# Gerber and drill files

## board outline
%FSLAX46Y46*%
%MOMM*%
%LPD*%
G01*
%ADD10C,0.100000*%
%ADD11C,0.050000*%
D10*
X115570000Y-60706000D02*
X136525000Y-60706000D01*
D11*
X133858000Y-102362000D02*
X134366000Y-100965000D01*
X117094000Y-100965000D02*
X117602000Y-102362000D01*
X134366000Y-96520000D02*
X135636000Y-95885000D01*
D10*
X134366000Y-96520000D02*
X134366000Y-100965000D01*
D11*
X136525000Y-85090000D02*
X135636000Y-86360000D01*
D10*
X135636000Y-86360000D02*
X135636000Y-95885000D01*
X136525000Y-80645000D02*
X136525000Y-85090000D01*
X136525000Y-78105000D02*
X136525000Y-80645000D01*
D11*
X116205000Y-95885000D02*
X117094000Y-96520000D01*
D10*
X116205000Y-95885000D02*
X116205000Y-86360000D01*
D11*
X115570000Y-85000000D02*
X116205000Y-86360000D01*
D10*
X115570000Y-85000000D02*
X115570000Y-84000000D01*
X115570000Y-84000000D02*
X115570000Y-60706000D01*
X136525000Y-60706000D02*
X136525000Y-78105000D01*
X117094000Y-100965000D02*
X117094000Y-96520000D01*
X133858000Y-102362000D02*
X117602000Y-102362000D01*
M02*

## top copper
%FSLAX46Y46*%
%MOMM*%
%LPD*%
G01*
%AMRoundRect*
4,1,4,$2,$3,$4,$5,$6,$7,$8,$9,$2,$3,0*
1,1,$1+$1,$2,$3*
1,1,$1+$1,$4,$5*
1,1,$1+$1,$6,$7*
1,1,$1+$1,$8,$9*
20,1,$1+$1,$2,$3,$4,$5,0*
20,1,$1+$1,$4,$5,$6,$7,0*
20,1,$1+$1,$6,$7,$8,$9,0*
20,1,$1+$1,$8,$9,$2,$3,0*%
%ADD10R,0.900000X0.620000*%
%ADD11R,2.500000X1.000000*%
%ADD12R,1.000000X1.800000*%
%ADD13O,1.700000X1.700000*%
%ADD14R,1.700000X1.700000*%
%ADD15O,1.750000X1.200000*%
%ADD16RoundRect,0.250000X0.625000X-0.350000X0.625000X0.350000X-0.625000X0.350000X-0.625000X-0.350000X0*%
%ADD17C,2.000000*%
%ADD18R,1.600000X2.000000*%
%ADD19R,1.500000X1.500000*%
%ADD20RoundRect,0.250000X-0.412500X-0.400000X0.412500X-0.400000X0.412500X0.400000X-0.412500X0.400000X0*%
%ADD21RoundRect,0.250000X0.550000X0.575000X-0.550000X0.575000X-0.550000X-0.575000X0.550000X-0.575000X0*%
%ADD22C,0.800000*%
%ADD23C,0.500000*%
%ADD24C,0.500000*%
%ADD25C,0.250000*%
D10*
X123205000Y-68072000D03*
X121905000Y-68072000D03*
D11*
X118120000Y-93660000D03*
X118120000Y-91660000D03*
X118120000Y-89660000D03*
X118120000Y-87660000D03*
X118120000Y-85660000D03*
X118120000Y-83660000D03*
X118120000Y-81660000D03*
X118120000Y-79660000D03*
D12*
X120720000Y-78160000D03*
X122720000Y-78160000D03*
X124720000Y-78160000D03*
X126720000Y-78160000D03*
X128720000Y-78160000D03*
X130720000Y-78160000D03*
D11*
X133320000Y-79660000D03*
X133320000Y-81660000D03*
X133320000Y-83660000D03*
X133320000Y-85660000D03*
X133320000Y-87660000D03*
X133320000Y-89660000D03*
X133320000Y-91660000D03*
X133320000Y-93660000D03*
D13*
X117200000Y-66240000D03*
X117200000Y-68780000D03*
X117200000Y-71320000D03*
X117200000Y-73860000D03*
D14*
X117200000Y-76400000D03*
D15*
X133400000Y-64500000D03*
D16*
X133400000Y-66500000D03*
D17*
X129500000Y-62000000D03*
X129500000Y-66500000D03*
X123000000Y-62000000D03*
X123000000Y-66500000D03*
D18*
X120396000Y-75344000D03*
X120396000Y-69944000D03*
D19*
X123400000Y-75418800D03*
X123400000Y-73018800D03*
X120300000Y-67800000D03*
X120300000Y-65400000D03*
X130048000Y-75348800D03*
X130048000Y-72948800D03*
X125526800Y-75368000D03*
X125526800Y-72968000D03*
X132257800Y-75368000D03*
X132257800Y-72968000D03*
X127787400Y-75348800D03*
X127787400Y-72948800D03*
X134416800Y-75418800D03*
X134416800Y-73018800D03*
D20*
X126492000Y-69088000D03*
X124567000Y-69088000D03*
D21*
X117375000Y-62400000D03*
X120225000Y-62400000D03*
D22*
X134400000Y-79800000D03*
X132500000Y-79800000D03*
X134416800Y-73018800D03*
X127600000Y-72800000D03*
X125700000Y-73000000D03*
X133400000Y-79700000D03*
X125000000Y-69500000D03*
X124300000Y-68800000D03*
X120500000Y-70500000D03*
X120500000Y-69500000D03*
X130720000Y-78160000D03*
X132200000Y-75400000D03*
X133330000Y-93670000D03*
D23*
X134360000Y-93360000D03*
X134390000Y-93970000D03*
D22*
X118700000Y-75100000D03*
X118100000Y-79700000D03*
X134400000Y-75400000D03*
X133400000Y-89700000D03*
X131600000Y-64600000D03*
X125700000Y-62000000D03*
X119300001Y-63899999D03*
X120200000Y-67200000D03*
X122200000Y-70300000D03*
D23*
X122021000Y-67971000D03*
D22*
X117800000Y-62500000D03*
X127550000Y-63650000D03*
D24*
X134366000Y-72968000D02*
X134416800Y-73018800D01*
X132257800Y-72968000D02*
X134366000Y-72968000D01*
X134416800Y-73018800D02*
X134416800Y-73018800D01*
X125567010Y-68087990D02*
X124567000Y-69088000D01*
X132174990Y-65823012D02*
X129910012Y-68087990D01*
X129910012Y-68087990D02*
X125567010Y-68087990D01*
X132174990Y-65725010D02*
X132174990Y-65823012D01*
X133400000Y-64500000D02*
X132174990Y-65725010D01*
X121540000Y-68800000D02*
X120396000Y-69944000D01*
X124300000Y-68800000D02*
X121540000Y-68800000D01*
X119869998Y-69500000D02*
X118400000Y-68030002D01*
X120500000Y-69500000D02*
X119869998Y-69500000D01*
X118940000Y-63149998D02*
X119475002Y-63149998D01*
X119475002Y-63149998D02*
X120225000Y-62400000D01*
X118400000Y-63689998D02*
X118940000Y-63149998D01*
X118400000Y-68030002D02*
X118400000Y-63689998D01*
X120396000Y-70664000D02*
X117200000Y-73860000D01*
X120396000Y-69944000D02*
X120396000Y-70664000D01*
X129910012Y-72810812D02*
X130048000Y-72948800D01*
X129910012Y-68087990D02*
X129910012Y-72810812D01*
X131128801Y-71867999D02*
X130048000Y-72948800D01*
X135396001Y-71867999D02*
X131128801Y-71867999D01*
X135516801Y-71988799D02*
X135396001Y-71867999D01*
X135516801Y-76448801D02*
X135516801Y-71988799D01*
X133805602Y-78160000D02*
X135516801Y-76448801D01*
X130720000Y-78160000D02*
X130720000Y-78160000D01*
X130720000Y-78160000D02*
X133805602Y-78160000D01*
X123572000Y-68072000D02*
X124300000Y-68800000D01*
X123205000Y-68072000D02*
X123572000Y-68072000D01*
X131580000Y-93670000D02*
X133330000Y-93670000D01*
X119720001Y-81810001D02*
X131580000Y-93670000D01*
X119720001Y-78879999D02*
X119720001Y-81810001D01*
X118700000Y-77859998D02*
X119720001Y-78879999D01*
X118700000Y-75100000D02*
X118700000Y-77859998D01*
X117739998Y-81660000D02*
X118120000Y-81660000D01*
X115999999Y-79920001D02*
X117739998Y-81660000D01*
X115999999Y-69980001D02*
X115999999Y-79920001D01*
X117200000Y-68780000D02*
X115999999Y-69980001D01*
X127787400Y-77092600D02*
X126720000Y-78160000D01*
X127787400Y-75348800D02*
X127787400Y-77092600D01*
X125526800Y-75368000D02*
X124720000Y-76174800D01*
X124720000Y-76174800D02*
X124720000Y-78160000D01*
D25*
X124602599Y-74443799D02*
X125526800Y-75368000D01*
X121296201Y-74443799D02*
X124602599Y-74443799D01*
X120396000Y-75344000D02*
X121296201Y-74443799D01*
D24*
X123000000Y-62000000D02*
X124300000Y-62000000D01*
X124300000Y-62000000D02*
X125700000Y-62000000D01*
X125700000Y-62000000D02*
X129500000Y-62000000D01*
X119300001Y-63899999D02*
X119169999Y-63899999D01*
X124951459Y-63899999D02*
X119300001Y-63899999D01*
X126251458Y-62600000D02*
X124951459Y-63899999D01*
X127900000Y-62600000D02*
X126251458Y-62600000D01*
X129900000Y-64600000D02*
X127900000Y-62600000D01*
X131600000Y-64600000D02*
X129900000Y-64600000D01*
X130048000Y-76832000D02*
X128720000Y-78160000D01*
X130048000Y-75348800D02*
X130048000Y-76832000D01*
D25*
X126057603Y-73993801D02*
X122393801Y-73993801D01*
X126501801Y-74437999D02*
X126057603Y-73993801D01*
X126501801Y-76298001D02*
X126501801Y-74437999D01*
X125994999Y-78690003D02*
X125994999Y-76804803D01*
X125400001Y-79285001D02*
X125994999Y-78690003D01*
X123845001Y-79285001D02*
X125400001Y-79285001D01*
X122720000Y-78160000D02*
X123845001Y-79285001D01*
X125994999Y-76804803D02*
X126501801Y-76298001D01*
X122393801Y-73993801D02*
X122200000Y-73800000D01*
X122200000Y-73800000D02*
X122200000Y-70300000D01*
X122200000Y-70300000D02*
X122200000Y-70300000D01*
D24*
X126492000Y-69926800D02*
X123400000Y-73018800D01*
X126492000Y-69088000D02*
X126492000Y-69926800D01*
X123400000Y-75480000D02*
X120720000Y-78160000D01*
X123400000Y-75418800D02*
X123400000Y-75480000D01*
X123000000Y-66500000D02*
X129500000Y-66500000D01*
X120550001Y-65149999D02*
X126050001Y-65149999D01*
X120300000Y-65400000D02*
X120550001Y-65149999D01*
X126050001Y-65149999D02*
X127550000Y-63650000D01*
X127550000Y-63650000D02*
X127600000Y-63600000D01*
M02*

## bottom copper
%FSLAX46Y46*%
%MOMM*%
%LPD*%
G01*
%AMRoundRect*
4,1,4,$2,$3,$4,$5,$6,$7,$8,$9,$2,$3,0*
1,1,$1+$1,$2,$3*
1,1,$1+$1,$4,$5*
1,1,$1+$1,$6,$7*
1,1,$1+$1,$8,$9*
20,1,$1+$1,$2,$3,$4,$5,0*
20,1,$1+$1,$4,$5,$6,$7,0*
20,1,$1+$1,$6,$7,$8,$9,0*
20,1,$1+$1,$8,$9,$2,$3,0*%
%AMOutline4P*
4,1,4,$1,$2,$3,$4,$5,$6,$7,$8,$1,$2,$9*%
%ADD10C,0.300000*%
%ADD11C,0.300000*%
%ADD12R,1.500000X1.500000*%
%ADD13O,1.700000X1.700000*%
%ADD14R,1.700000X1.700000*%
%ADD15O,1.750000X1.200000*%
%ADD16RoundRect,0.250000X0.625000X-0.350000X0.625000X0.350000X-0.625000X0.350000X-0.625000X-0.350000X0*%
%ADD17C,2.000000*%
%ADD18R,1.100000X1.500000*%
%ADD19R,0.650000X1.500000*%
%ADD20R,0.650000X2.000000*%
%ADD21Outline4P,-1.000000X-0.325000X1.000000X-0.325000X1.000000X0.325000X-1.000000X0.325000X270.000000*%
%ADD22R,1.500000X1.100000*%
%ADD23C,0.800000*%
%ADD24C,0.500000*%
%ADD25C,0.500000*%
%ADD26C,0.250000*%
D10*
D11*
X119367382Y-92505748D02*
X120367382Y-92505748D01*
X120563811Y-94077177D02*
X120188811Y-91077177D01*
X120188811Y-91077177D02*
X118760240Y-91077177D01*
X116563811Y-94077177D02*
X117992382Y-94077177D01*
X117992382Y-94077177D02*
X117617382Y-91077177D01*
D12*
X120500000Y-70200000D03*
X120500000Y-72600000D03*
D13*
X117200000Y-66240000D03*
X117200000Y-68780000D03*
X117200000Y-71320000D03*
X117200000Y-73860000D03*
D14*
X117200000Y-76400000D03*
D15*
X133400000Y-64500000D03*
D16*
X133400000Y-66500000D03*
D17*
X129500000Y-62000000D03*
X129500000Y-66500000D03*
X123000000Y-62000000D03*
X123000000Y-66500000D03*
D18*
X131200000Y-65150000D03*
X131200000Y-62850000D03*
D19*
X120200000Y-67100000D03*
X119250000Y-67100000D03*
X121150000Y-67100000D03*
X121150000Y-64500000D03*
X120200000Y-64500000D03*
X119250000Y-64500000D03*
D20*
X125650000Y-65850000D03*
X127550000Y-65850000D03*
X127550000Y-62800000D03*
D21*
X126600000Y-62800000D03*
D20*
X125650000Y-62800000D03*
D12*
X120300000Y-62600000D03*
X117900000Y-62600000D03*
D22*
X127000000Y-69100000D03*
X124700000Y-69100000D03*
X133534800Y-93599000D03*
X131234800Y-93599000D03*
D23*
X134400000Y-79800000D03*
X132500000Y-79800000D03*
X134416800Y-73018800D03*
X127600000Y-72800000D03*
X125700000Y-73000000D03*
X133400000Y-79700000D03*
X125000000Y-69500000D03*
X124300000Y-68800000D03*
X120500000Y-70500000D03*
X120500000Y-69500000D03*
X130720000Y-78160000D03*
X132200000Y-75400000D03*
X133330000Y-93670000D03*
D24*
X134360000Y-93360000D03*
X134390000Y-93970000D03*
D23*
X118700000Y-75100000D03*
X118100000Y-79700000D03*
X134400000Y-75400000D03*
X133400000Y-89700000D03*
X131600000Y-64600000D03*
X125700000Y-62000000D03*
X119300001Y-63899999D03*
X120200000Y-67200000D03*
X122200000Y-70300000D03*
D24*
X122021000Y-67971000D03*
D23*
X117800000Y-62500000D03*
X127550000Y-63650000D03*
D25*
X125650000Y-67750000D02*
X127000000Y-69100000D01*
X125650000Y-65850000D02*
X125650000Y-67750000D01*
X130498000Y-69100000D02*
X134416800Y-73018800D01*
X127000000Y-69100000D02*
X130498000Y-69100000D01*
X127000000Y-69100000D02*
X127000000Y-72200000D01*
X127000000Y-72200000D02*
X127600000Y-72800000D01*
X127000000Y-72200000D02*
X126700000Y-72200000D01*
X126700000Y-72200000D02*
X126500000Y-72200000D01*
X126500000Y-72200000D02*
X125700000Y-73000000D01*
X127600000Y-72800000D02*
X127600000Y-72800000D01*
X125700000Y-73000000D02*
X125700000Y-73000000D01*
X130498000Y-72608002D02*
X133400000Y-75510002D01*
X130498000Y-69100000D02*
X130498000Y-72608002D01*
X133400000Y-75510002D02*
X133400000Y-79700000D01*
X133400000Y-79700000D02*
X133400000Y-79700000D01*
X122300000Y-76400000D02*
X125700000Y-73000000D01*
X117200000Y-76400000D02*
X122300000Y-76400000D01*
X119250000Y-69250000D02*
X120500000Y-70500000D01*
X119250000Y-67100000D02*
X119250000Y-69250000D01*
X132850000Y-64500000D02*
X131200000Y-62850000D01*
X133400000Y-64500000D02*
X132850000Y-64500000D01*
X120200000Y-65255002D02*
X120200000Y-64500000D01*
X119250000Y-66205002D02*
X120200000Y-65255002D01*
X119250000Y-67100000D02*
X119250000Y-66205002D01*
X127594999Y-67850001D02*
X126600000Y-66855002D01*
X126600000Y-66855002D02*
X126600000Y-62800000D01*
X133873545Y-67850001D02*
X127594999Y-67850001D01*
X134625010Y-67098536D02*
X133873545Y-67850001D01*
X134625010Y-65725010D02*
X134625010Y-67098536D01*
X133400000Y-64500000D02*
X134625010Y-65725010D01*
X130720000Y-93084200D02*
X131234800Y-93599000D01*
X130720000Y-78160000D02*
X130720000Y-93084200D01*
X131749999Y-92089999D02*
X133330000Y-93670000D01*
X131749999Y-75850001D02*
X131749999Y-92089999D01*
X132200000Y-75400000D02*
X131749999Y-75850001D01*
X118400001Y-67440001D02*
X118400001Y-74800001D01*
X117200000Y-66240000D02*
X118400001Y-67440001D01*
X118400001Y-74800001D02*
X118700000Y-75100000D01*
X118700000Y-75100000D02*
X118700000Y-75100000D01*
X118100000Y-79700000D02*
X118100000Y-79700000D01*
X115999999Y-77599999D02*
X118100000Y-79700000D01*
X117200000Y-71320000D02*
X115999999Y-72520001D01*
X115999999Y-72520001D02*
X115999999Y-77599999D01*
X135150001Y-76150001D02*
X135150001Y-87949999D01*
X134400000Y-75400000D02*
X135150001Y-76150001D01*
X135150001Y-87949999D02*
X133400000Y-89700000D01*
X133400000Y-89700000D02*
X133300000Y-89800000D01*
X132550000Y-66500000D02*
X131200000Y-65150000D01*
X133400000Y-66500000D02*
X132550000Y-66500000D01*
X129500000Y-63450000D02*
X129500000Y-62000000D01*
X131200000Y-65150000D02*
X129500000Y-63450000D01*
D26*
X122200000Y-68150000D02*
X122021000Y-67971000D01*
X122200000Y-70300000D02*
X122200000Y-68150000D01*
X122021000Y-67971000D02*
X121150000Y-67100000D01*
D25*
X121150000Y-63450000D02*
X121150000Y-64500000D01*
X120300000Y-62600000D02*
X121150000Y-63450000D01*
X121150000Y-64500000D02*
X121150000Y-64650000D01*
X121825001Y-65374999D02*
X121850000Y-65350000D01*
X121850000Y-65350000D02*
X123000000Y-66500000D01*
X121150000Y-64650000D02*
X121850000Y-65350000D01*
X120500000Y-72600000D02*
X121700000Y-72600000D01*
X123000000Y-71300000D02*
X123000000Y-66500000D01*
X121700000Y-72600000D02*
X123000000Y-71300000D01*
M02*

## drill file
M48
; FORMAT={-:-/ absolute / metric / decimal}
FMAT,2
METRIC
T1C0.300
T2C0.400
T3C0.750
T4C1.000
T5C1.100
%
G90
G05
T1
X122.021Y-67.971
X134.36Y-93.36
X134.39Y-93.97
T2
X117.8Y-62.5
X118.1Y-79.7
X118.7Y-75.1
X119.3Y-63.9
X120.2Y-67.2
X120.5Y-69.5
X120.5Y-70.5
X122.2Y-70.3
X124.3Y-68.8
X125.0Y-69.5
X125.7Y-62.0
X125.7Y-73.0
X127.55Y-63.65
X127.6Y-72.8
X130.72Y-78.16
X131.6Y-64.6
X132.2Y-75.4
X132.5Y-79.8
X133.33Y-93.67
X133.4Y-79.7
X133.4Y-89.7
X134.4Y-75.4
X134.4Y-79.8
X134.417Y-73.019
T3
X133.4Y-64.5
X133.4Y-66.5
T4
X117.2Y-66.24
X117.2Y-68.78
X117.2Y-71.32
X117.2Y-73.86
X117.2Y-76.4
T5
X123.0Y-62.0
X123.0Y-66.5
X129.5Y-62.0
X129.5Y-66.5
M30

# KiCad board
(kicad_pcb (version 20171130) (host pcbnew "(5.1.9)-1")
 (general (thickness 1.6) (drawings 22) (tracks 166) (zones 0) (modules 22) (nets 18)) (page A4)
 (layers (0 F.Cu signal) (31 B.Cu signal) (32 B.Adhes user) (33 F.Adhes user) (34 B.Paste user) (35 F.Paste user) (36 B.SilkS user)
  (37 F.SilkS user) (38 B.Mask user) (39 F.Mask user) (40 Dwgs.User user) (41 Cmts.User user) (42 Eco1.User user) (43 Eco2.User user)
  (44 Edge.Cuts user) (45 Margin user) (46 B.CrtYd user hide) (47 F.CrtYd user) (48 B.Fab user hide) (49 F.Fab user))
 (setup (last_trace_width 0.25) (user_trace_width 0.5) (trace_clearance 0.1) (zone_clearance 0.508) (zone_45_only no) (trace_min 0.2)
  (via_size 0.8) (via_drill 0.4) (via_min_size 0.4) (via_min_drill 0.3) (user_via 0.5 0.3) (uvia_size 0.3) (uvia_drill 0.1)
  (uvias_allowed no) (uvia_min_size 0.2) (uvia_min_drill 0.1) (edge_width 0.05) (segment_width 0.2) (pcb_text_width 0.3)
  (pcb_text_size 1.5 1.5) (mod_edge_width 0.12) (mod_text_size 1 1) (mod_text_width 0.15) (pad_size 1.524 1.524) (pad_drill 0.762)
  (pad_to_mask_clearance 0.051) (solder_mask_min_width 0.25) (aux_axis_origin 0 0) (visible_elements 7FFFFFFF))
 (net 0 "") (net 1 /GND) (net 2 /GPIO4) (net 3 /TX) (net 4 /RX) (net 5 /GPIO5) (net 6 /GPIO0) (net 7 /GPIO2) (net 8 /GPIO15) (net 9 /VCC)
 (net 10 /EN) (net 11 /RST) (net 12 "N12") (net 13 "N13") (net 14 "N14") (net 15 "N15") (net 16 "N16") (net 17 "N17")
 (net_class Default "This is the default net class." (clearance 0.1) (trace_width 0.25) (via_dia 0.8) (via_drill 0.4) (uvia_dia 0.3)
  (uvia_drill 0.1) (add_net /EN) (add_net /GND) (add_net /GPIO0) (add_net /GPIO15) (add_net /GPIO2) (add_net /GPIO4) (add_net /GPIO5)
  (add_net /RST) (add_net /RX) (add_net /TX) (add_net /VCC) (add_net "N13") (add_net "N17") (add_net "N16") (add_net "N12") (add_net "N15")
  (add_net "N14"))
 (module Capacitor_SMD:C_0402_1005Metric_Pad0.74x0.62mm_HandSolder (layer F.Cu) (at 122.555 68.072)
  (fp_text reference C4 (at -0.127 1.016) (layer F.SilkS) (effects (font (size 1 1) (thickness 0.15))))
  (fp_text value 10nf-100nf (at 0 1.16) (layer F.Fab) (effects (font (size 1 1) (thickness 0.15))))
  (pad 2 smd rect (at 0.65 0) (size 0.9 0.62) (layers F.Cu F.Paste F.Mask) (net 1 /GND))
  (pad 1 smd rect (at -0.65 0) (size 0.9 0.62) (layers F.Cu F.Paste F.Mask) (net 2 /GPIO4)))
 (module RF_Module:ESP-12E (layer F.Cu) (at 125.72 90.16 180)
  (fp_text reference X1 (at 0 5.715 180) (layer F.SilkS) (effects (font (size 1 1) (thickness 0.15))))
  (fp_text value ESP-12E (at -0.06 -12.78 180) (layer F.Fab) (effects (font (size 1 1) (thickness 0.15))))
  (pad 22 smd rect (at 7.6 -3.5 180) (size 2.5 1) (layers F.Cu F.Paste F.Mask))
  (pad 21 smd rect (at 7.6 -1.5 180) (size 2.5 1) (layers F.Cu F.Paste F.Mask))
  (pad 20 smd rect (at 7.6 0.5 180) (size 2.5 1) (layers F.Cu F.Paste F.Mask))
  (pad 19 smd rect (at 7.6 2.5 180) (size 2.5 1) (layers F.Cu F.Paste F.Mask))
  (pad 18 smd rect (at 7.6 4.5 180) (size 2.5 1) (layers F.Cu F.Paste F.Mask))
  (pad 17 smd rect (at 7.6 6.5 180) (size 2.5 1) (layers F.Cu F.Paste F.Mask))
  (pad 16 smd rect (at 7.6 8.5 180) (size 2.5 1) (layers F.Cu F.Paste F.Mask) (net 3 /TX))
  (pad 15 smd rect (at 7.6 10.5 180) (size 2.5 1) (layers F.Cu F.Paste F.Mask) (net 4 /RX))
  (pad 14 smd rect (at 5 12 180) (size 1 1.8) (layers F.Cu F.Paste F.Mask) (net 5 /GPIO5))
  (pad 13 smd rect (at 3 12 180) (size 1 1.8) (layers F.Cu F.Paste F.Mask) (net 2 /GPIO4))
  (pad 12 smd rect (at 1 12 180) (size 1 1.8) (layers F.Cu F.Paste F.Mask) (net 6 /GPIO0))
  (pad 11 smd rect (at -1 12 180) (size 1 1.8) (layers F.Cu F.Paste F.Mask) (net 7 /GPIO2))
  (pad 10 smd rect (at -3 12 180) (size 1 1.8) (layers F.Cu F.Paste F.Mask) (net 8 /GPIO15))
  (pad 9 smd rect (at -5 12 180) (size 1 1.8) (layers F.Cu F.Paste F.Mask) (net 1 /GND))
  (pad 8 smd rect (at -7.6 10.5 180) (size 2.5 1) (layers F.Cu F.Paste F.Mask) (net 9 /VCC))
  (pad 7 smd rect (at -7.6 8.5 180) (size 2.5 1) (layers F.Cu F.Paste F.Mask))
  (pad 6 smd rect (at -7.6 6.5 180) (size 2.5 1) (layers F.Cu F.Paste F.Mask))
  (pad 5 smd rect (at -7.6 4.5 180) (size 2.5 1) (layers F.Cu F.Paste F.Mask))
  (pad 4 smd rect (at -7.6 2.5 180) (size 2.5 1) (layers F.Cu F.Paste F.Mask))
  (pad 3 smd rect (at -7.6 0.5 180) (size 2.5 1) (layers F.Cu F.Paste F.Mask) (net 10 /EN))
  (pad 2 smd rect (at -7.6 -1.5 180) (size 2.5 1) (layers F.Cu F.Paste F.Mask))
  (pad 1 smd rect (at -7.6 -3.5 180) (size 2.5 1) (layers F.Cu F.Paste F.Mask) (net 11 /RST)))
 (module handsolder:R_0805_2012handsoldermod (layer B.Cu) (at 120.5 71.4 90)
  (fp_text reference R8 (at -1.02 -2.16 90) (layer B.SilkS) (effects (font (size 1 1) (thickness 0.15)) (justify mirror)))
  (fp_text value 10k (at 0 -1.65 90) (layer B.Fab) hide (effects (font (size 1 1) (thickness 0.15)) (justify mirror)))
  (pad 2 smd rect (at 1.2 0 90) (size 1.5 1.5) (layers B.Cu B.Paste B.Mask) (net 1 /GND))
  (pad 1 smd rect (at -1.2 0 90) (size 1.5 1.5) (layers B.Cu B.Paste B.Mask) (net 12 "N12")))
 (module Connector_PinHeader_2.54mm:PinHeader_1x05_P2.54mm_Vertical (layer F.Cu) (at 117.2 76.4 180)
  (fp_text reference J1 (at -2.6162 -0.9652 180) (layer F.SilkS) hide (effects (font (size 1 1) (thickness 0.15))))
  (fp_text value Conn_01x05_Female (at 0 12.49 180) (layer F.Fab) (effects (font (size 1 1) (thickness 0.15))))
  (pad 5 thru_hole oval (at 0 10.16 180) (size 1.7 1.7) (drill 1) (layers *.Cu *.Mask) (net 11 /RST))
  (pad 4 thru_hole oval (at 0 7.62 180) (size 1.7 1.7) (drill 1) (layers *.Cu *.Mask) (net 3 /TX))
  (pad 3 thru_hole oval (at 0 5.08 180) (size 1.7 1.7) (drill 1) (layers *.Cu *.Mask) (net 4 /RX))
  (pad 2 thru_hole oval (at 0 2.54 180) (size 1.7 1.7) (drill 1) (layers *.Cu *.Mask) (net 1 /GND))
  (pad 1 thru_hole rect (at 0 0 180) (size 1.7 1.7) (drill 1) (layers *.Cu *.Mask) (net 9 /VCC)))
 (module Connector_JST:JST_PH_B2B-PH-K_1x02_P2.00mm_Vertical (layer F.Cu) (at 133.4 66.5 90)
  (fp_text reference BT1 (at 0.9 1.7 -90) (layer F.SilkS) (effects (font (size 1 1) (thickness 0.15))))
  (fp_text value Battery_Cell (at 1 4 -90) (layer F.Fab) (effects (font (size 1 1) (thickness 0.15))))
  (pad 2 thru_hole oval (at 2 0 90) (size 1.2 1.75) (drill 0.75) (layers *.Cu *.Mask) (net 1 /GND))
  (pad 1 thru_hole roundrect (at 0 0 90) (size 1.2 1.75) (drill 0.75) (layers *.Cu *.Mask) (roundrect_rratio 0.208333) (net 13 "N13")))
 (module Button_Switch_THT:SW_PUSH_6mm (layer F.Cu) (at 123 62)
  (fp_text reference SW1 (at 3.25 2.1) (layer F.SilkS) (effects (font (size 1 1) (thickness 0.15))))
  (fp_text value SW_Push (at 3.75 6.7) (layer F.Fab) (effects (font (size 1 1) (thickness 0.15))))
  (pad 1 thru_hole circle (at 6.5 0 90) (size 2 2) (drill 1.1) (layers *.Cu *.Mask) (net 13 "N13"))
  (pad 2 thru_hole circle (at 6.5 4.5 90) (size 2 2) (drill 1.1) (layers *.Cu *.Mask) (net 12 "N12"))
  (pad 1 thru_hole circle (at 0 0 90) (size 2 2) (drill 1.1) (layers *.Cu *.Mask) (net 13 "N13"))
  (pad 2 thru_hole circle (at 0 4.5 90) (size 2 2) (drill 1.1) (layers *.Cu *.Mask) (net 12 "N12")))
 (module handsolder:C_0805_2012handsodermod (layer B.Cu) (at 131.2 64 270)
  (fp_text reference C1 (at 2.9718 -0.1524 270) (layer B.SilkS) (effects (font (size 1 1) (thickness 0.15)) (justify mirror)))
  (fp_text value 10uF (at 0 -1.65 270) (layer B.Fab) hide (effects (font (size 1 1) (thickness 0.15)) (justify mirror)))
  (pad 2 smd rect (at 1.15 0 270) (size 1.5 1.1) (layers B.Cu B.Paste B.Mask) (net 13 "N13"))
  (pad 1 smd rect (at -1.15 0 270) (size 1.5 1.1) (layers B.Cu B.Paste B.Mask) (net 1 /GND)))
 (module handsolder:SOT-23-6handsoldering (layer B.Cu) (at 120.2 65.8 270)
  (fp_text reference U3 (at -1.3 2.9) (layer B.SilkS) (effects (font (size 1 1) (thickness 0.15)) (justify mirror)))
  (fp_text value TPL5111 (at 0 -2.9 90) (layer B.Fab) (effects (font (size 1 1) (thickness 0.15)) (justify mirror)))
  (pad 5 smd rect (at 1.3 0 270) (size 1.5 0.65) (layers B.Cu B.Paste B.Mask) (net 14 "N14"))
  (pad 6 smd rect (at 1.3 0.95 270) (size 1.5 0.65) (layers B.Cu B.Paste B.Mask) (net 1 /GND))
  (pad 4 smd rect (at 1.3 -0.95 270) (size 1.5 0.65) (layers B.Cu B.Paste B.Mask) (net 2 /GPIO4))
  (pad 3 smd rect (at -1.3 -0.95 270) (size 1.5 0.65) (layers B.Cu B.Paste B.Mask) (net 12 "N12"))
  (pad 2 smd rect (at -1.3 0 270) (size 1.5 0.65) (layers B.Cu B.Paste B.Mask) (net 1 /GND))
  (pad 1 smd rect (at -1.3 0.95 270) (size 1.5 0.65) (layers B.Cu B.Paste B.Mask) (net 13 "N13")))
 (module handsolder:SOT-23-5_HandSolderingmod (layer B.Cu) (at 126.6 64.35 270)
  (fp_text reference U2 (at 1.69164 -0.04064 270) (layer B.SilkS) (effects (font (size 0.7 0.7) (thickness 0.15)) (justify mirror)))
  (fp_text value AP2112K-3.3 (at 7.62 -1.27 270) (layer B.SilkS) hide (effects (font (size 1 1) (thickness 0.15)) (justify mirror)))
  (pad 5 smd rect (at 1.5 0.95 270) (size 2 0.65) (layers B.Cu B.Paste B.Mask) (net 9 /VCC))
  (pad 4 smd rect (at 1.5 -0.95 270) (size 2 0.65) (layers B.Cu B.Paste B.Mask))
  (pad 3 smd rect (at -1.55 -0.95 270) (size 2 0.65) (layers B.Cu B.Paste B.Mask) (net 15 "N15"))
  (pad 2 smd trapezoid (at -1.55 0 270) (size 2 0.65) (layers B.Cu B.Paste B.Mask) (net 1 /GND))
  (pad 1 smd rect (at -1.55 0.95 270) (size 2 0.65) (layers B.Cu B.Paste B.Mask) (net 13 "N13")))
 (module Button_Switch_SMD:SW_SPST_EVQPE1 (layer F.Cu) (at 120.396 72.644 90)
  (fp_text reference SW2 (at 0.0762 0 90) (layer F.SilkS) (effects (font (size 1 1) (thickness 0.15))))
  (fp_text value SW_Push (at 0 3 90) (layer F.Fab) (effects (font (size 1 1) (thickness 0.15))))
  (pad 1 smd rect (at -2.7 0 90) (size 2 1.6) (layers F.Cu F.Paste F.Mask) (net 6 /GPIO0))
  (pad 2 smd rect (at 2.7 0 90) (size 2 1.6) (layers F.Cu F.Paste F.Mask) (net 1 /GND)))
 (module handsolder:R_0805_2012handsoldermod (layer F.Cu) (at 123.4 74.2188 270)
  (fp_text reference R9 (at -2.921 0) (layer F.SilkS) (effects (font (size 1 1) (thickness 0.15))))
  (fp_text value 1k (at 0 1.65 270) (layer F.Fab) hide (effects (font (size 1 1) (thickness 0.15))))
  (pad 2 smd rect (at 1.2 0 270) (size 1.5 1.5) (layers F.Cu F.Paste F.Mask) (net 5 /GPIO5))
  (pad 1 smd rect (at -1.2 0 270) (size 1.5 1.5) (layers F.Cu F.Paste F.Mask) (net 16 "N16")))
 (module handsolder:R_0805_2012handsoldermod (layer F.Cu) (at 120.3 66.6 270)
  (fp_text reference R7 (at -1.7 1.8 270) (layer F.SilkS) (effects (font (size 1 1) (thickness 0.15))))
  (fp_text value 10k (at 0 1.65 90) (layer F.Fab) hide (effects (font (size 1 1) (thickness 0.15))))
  (pad 2 smd rect (at 1.2 0 270) (size 1.5 1.5) (layers F.Cu F.Paste F.Mask) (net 14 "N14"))
  (pad 1 smd rect (at -1.2 0 270) (size 1.5 1.5) (layers F.Cu F.Paste F.Mask) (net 15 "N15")))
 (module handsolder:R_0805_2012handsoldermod (layer B.Cu) (at 119.1 62.6)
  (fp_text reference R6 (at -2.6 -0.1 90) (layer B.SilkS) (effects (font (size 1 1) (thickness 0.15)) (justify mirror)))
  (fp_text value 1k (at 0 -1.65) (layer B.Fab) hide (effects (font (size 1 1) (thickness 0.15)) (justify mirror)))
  (pad 2 smd rect (at 1.2 0) (size 1.5 1.5) (layers B.Cu B.Paste B.Mask) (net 12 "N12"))
  (pad 1 smd rect (at -1.2 0) (size 1.5 1.5) (layers B.Cu B.Paste B.Mask) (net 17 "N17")))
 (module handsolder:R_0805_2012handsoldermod (layer F.Cu) (at 130.048 74.1488 270)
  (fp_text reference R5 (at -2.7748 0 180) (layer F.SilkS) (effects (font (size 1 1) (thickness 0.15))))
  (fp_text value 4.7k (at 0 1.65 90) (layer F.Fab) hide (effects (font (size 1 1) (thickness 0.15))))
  (pad 2 smd rect (at 1.2 0 270) (size 1.5 1.5) (layers F.Cu F.Paste F.Mask) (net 8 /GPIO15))
  (pad 1 smd rect (at -1.2 0 270) (size 1.5 1.5) (layers F.Cu F.Paste F.Mask) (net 1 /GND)))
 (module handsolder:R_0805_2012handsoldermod (layer F.Cu) (at 125.5268 74.168 270)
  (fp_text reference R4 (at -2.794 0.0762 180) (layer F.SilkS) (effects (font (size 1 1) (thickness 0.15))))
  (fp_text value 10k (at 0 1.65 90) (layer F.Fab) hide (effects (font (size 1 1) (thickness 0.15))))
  (pad 2 smd rect (at 1.2 0 270) (size 1.5 1.5) (layers F.Cu F.Paste F.Mask) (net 6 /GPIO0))
  (pad 1 smd rect (at -1.2 0 270) (size 1.5 1.5) (layers F.Cu F.Paste F.Mask) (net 9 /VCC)))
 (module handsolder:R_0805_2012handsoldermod (layer F.Cu) (at 132.2578 74.168 270)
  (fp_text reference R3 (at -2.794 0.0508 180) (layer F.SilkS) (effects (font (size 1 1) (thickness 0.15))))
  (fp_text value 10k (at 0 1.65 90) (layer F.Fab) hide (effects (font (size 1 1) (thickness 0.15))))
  (pad 2 smd rect (at 1.2 0 270) (size 1.5 1.5) (layers F.Cu F.Paste F.Mask) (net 11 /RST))
  (pad 1 smd rect (at -1.2 0 270) (size 1.5 1.5) (layers F.Cu F.Paste F.Mask) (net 9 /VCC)))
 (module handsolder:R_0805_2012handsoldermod (layer F.Cu) (at 127.7874 74.1488 270)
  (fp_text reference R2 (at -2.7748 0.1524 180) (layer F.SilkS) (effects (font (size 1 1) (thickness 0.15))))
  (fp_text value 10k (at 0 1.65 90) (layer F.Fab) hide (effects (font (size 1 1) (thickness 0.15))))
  (pad 2 smd rect (at 1.2 0 270) (size 1.5 1.5) (layers F.Cu F.Paste F.Mask) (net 7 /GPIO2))
  (pad 1 smd rect (at -1.2 0 270) (size 1.5 1.5) (layers F.Cu F.Paste F.Mask) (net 9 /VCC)))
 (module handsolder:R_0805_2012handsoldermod (layer F.Cu) (at 134.4168 74.2188 270)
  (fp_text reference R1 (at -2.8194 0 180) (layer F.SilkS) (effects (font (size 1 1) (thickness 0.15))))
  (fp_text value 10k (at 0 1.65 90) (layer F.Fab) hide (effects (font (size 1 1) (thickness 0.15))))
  (pad 2 smd rect (at 1.2 0 270) (size 1.5 1.5) (layers F.Cu F.Paste F.Mask) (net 10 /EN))
  (pad 1 smd rect (at -1.2 0 270) (size 1.5 1.5) (layers F.Cu F.Paste F.Mask) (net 9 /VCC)))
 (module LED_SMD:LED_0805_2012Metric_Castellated (layer F.Cu) (at 125.5295 69.088)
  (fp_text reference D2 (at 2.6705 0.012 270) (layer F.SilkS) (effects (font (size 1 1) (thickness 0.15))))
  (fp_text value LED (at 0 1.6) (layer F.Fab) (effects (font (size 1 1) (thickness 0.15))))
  (pad 2 smd roundrect (at 0.9625 0) (size 1.325 1.3) (layers F.Cu F.Paste F.Mask) (roundrect_rratio 0.1923076923076923) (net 16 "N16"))
  (pad 1 smd roundrect (at -0.9625 0) (size 1.325 1.3) (layers F.Cu F.Paste F.Mask) (roundrect_rratio 0.1923076923076923) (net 1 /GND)))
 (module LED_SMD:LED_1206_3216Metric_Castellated (layer F.Cu) (at 118.8 62.4 180)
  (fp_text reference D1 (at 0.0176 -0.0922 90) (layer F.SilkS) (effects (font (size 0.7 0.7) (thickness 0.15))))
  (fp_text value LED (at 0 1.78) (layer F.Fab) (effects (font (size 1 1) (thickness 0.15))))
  (pad 2 smd roundrect (at 1.425 0 180) (size 1.6 1.65) (layers F.Cu F.Paste F.Mask) (roundrect_rratio 0.15625) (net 17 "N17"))
  (pad 1 smd roundrect (at -1.425 0 180) (size 1.6 1.65) (layers F.Cu F.Paste F.Mask) (roundrect_rratio 0.15625) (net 1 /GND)))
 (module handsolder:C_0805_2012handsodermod (layer B.Cu) (at 125.85 69.1)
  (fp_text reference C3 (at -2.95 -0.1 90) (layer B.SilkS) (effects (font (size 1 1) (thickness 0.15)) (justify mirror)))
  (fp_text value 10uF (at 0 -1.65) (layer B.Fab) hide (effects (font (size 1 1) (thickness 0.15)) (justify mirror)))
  (pad 2 smd rect (at 1.15 0) (size 1.5 1.1) (layers B.Cu B.Paste B.Mask) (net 9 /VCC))
  (pad 1 smd rect (at -1.15 0) (size 1.5 1.1) (layers B.Cu B.Paste B.Mask) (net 1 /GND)))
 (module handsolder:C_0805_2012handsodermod (layer B.Cu) (at 132.3848 93.599)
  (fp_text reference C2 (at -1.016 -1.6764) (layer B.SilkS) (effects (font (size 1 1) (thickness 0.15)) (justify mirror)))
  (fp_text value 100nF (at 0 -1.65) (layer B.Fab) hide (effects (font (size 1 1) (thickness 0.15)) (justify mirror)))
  (pad 2 smd rect (at 1.15 0) (size 1.5 1.1) (layers B.Cu B.Paste B.Mask) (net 11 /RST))
  (pad 1 smd rect (at -1.15 0) (size 1.5 1.1) (layers B.Cu B.Paste B.Mask) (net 1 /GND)))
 (gr_line (start 115.57 60.706) (end 136.525 60.706) (layer Edge.Cuts) (width 0.1))
 (gr_line (start 133.858 102.362) (end 134.366 100.965) (layer Edge.Cuts) (width 0.05))
 (gr_line (start 117.094 100.965) (end 117.602 102.362) (layer Edge.Cuts) (width 0.05))
 (gr_line (start 134.366 96.52) (end 135.636 95.885) (layer Edge.Cuts) (width 0.05))
 (gr_line (start 134.366 96.52) (end 134.366 100.965) (layer Edge.Cuts) (width 0.1))
 (gr_line (start 136.525 85.09) (end 135.636 86.36) (layer Edge.Cuts) (width 0.05))
 (gr_line (start 135.636 86.36) (end 135.636 95.885) (layer Edge.Cuts) (width 0.1))
 (gr_line (start 136.525 80.645) (end 136.525 85.09) (layer Edge.Cuts) (width 0.1))
 (gr_line (start 136.525 78.105) (end 136.525 80.645) (layer Edge.Cuts) (width 0.1))
 (gr_line (start 116.205 95.885) (end 117.094 96.52) (layer Edge.Cuts) (width 0.05))
 (gr_line (start 116.205 95.885) (end 116.205 86.36) (layer Edge.Cuts) (width 0.1))
 (gr_line (start 115.57 85) (end 116.205 86.36) (layer Edge.Cuts) (width 0.05))
 (gr_line (start 115.57 85) (end 115.57 84) (layer Edge.Cuts) (width 0.1))
 (gr_line (start 115.57 84) (end 115.57 60.706) (layer Edge.Cuts) (width 0.1))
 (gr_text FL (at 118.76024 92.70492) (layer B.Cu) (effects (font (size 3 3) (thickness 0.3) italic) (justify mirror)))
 (gr_line (start 136.525 60.706) (end 136.525 78.105) (layer Edge.Cuts) (width 0.1))
 (gr_line (start 117.094 100.965) (end 117.094 96.52) (layer Edge.Cuts) (width 0.1))
 (gr_line (start 133.858 102.362) (end 117.602 102.362) (layer Edge.Cuts) (width 0.1))
 (via (at 134.4 79.8) (size 0.8) (drill 0.4) (layers F.Cu B.Cu) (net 9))
 (via (at 132.5 79.8) (size 0.8) (drill 0.4) (layers F.Cu B.Cu) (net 9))
 (segment (start 125.65 67.75) (end 127 69.1) (width 0.5) (layer B.Cu) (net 9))
 (segment (start 125.65 65.85) (end 125.65 67.75) (width 0.5) (layer B.Cu) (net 9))
 (segment (start 134.366 72.968) (end 134.4168 73.0188) (width 0.5) (layer F.Cu) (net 9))
 (segment (start 132.2578 72.968) (end 134.366 72.968) (width 0.5) (layer F.Cu) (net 9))
 (segment (start 134.4168 73.0188) (end 134.4168 73.0188) (width 0.5) (layer F.Cu) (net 9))
 (via (at 134.4168 73.0188) (size 0.8) (drill 0.4) (layers F.Cu B.Cu) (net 9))
 (segment (start 130.498 69.1) (end 134.4168 73.0188) (width 0.5) (layer B.Cu) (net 9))
 (segment (start 127 69.1) (end 130.498 69.1) (width 0.5) (layer B.Cu) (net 9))
 (segment (start 127 69.1) (end 127 72.2) (width 0.5) (layer B.Cu) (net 9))
 (segment (start 127 72.2) (end 127.6 72.8) (width 0.5) (layer B.Cu) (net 9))
 (segment (start 127 72.2) (end 126.7 72.2) (width 0.5) (layer B.Cu) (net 9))
 (segment (start 126.7 72.2) (end 126.5 72.2) (width 0.5) (layer B.Cu) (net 9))
 (segment (start 126.5 72.2) (end 125.7 73) (width 0.5) (layer B.Cu) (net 9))
 (segment (start 127.6 72.8) (end 127.6 72.8) (width 0.5) (layer B.Cu) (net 9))
 (via (at 127.6 72.8) (size 0.8) (drill 0.4) (layers F.Cu B.Cu) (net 9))
 (segment (start 125.7 73) (end 125.7 73) (width 0.5) (layer B.Cu) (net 9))
 (via (at 125.7 73) (size 0.8) (drill 0.4) (layers F.Cu B.Cu) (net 9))
 (segment (start 130.498 72.608002) (end 133.4 75.510002) (width 0.5) (layer B.Cu) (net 9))
 (segment (start 130.498 69.1) (end 130.498 72.608002) (width 0.5) (layer B.Cu) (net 9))
 (segment (start 133.4 75.510002) (end 133.4 79.7) (width 0.5) (layer B.Cu) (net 9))
 (segment (start 133.4 79.7) (end 133.4 79.7) (width 0.5) (layer B.Cu) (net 9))
 (via (at 133.4 79.7) (size 0.8) (drill 0.4) (layers F.Cu B.Cu) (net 9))
 (segment (start 122.3 76.4) (end 125.7 73) (width 0.5) (layer B.Cu) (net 9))
 (segment (start 117.2 76.4) (end 122.3 76.4) (width 0.5) (layer B.Cu) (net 9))
 (via (at 125 69.5) (size 0.8) (drill 0.4) (layers F.Cu B.Cu) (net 1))
 (via (at 124.3 68.8) (size 0.8) (drill 0.4) (layers F.Cu B.Cu) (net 1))
 (via (at 120.5 70.5) (size 0.8) (drill 0.4) (layers F.Cu B.Cu) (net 1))
 (via (at 120.5 69.5) (size 0.8) (drill 0.4) (layers F.Cu B.Cu) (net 1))
 (segment (start 119.25 69.25) (end 120.5 70.5) (width 0.5) (layer B.Cu) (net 1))
 (segment (start 119.25 67.1) (end 119.25 69.25) (width 0.5) (layer B.Cu) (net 1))
 (segment (start 132.85 64.5) (end 131.2 62.85) (width 0.5) (layer B.Cu) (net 1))
 (segment (start 133.4 64.5) (end 132.85 64.5) (width 0.5) (layer B.Cu) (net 1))
 (segment (start 120.2 65.255002) (end 120.2 64.5) (width 0.5) (layer B.Cu) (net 1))
 (segment (start 119.25 66.205002) (end 120.2 65.255002) (width 0.5) (layer B.Cu) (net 1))
 (segment (start 119.25 67.1) (end 119.25 66.205002) (width 0.5) (layer B.Cu) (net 1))
 (segment (start 127.594999 67.850001) (end 126.6 66.855002) (width 0.5) (layer B.Cu) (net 1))
 (segment (start 126.6 66.855002) (end 126.6 62.8) (width 0.5) (layer B.Cu) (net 1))
 (segment (start 133.873545 67.850001) (end 127.594999 67.850001) (width 0.5) (layer B.Cu) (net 1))
 (segment (start 134.62501 67.098536) (end 133.873545 67.850001) (width 0.5) (layer B.Cu) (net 1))
 (segment (start 134.62501 65.72501) (end 134.62501 67.098536) (width 0.5) (layer B.Cu) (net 1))
 (segment (start 133.4 64.5) (end 134.62501 65.72501) (width 0.5) (layer B.Cu) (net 1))
 (segment (start 125.56701 68.08799) (end 124.567 69.088) (width 0.5) (layer F.Cu) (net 1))
 (segment (start 132.17499 65.823012) (end 129.910012 68.08799) (width 0.5) (layer F.Cu) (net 1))
 (segment (start 129.910012 68.08799) (end 125.56701 68.08799) (width 0.5) (layer F.Cu) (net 1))
 (segment (start 132.17499 65.72501) (end 132.17499 65.823012) (width 0.5) (layer F.Cu) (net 1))
 (segment (start 133.4 64.5) (end 132.17499 65.72501) (width 0.5) (layer F.Cu) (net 1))
 (segment (start 121.54 68.8) (end 120.396 69.944) (width 0.5) (layer F.Cu) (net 1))
 (segment (start 124.3 68.8) (end 121.54 68.8) (width 0.5) (layer F.Cu) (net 1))
 (segment (start 119.869998 69.5) (end 118.4 68.030002) (width 0.5) (layer F.Cu) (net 1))
 (segment (start 120.5 69.5) (end 119.869998 69.5) (width 0.5) (layer F.Cu) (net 1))
 (segment (start 118.94 63.149998) (end 119.475002 63.149998) (width 0.5) (layer F.Cu) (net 1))
 (segment (start 119.475002 63.149998) (end 120.225 62.4) (width 0.5) (layer F.Cu) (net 1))
 (segment (start 118.4 63.689998) (end 118.94 63.149998) (width 0.5) (layer F.Cu) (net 1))
 (segment (start 118.4 68.030002) (end 118.4 63.689998) (width 0.5) (layer F.Cu) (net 1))
 (segment (start 120.396 70.664) (end 117.2 73.86) (width 0.5) (layer F.Cu) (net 1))
 (segment (start 120.396 69.944) (end 120.396 70.664) (width 0.5) (layer F.Cu) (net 1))
 (segment (start 129.910012 72.810812) (end 130.048 72.9488) (width 0.5) (layer F.Cu) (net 1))
 (segment (start 129.910012 68.08799) (end 129.910012 72.810812) (width 0.5) (layer F.Cu) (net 1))
 (segment (start 131.128801 71.867999) (end 130.048 72.9488) (width 0.5) (layer F.Cu) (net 1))
 (segment (start 135.396001 71.867999) (end 131.128801 71.867999) (width 0.5) (layer F.Cu) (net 1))
 (segment (start 135.516801 71.988799) (end 135.396001 71.867999) (width 0.5) (layer F.Cu) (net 1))
 (segment (start 135.516801 76.448801) (end 135.516801 71.988799) (width 0.5) (layer F.Cu) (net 1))
 (segment (start 133.805602 78.16) (end 135.516801 76.448801) (width 0.5) (layer F.Cu) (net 1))
 (segment (start 130.72 78.16) (end 130.72 78.16) (width 0.5) (layer F.Cu) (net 1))
 (segment (start 130.72 78.16) (end 133.805602 78.16) (width 0.5) (layer F.Cu) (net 1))
 (via (at 130.72 78.16) (size 0.8) (drill 0.4) (layers F.Cu B.Cu) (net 1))
 (segment (start 130.72 93.0842) (end 131.2348 93.599) (width 0.5) (layer B.Cu) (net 1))
 (segment (start 130.72 78.16) (end 130.72 93.0842) (width 0.5) (layer B.Cu) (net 1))
 (segment (start 123.572 68.072) (end 124.3 68.8) (width 0.5) (layer F.Cu) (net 1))
 (segment (start 123.205 68.072) (end 123.572 68.072) (width 0.5) (layer F.Cu) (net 1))
 (via (at 132.2 75.4) (size 0.8) (drill 0.4) (layers F.Cu B.Cu) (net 11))
 (via (at 133.33 93.67) (size 0.8) (drill 0.4) (layers F.Cu B.Cu) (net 11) (status 30))
 (via (at 134.36 93.36) (size 0.5) (drill 0.3) (layers F.Cu B.Cu) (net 11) (status 30))
 (via (at 134.39 93.97) (size 0.5) (drill 0.3) (layers F.Cu B.Cu) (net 11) (status 30))
 (segment (start 131.749999 92.089999) (end 133.33 93.67) (width 0.5) (layer B.Cu) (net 11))
 (segment (start 131.749999 75.850001) (end 131.749999 92.089999) (width 0.5) (layer B.Cu) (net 11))
 (segment (start 132.2 75.4) (end 131.749999 75.850001) (width 0.5) (layer B.Cu) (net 11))
 (segment (start 118.400001 67.440001) (end 118.400001 74.800001) (width 0.5) (layer B.Cu) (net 11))
 (segment (start 117.2 66.24) (end 118.400001 67.440001) (width 0.5) (layer B.Cu) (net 11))
 (segment (start 118.400001 74.800001) (end 118.7 75.1) (width 0.5) (layer B.Cu) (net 11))
 (segment (start 118.7 75.1) (end 118.7 75.1) (width 0.5) (layer B.Cu) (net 11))
 (via (at 118.7 75.1) (size 0.8) (drill 0.4) (layers F.Cu B.Cu) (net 11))
 (segment (start 131.58 93.67) (end 133.33 93.67) (width 0.5) (layer F.Cu) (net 11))
 (segment (start 119.720001 81.810001) (end 131.58 93.67) (width 0.5) (layer F.Cu) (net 11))
 (segment (start 119.720001 78.879999) (end 119.720001 81.810001) (width 0.5) (layer F.Cu) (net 11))
 (segment (start 118.7 77.859998) (end 119.720001 78.879999) (width 0.5) (layer F.Cu) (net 11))
 (segment (start 118.7 75.1) (end 118.7 77.859998) (width 0.5) (layer F.Cu) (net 11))
 (segment (start 118.1 79.7) (end 118.1 79.7) (width 0.5) (layer B.Cu) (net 4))
 (via (at 118.1 79.7) (size 0.8) (drill 0.4) (layers F.Cu B.Cu) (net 4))
 (segment (start 115.999999 77.599999) (end 118.1 79.7) (width 0.5) (layer B.Cu) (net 4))
 (segment (start 117.2 71.32) (end 115.999999 72.520001) (width 0.5) (layer B.Cu) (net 4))
 (segment (start 115.999999 72.520001) (end 115.999999 77.599999) (width 0.5) (layer B.Cu) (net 4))
 (segment (start 117.739998 81.66) (end 118.12 81.66) (width 0.5) (layer F.Cu) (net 3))
 (segment (start 115.999999 79.920001) (end 117.739998 81.66) (width 0.5) (layer F.Cu) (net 3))
 (segment (start 115.999999 69.980001) (end 115.999999 79.920001) (width 0.5) (layer F.Cu) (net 3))
 (segment (start 117.2 68.78) (end 115.999999 69.980001) (width 0.5) (layer F.Cu) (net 3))
 (via (at 134.4 75.4) (size 0.8) (drill 0.4) (layers F.Cu B.Cu) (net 10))
 (segment (start 135.150001 76.150001) (end 135.150001 87.949999) (width 0.5) (layer B.Cu) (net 10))
 (segment (start 134.4 75.4) (end 135.150001 76.150001) (width 0.5) (layer B.Cu) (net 10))
 (segment (start 135.150001 87.949999) (end 133.4 89.7) (width 0.5) (layer B.Cu) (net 10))
 (segment (start 133.4 89.7) (end 133.3 89.8) (width 0.5) (layer B.Cu) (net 10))
 (via (at 133.4 89.7) (size 0.8) (drill 0.4) (layers F.Cu B.Cu) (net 10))
 (segment (start 127.7874 77.0926) (end 126.72 78.16) (width 0.5) (layer F.Cu) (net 7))
 (segment (start 127.7874 75.3488) (end 127.7874 77.0926) (width 0.5) (layer F.Cu) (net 7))
 (segment (start 125.5268 75.368) (end 124.72 76.1748) (width 0.5) (layer F.Cu) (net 6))
 (segment (start 124.72 76.1748) (end 124.72 78.16) (width 0.5) (layer F.Cu) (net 6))
 (segment (start 124.602599 74.443799) (end 125.5268 75.368) (width 0.25) (layer F.Cu) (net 6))
 (segment (start 121.296201 74.443799) (end 124.602599 74.443799) (width 0.25) (layer F.Cu) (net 6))
 (segment (start 120.396 75.344) (end 121.296201 74.443799) (width 0.25) (layer F.Cu) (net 6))
 (via (at 131.6 64.6) (size 0.8) (drill 0.4) (layers F.Cu B.Cu) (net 13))
 (segment (start 123 62) (end 124.3 62) (width 0.5) (layer F.Cu) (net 13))
 (segment (start 124.3 62) (end 125.7 62) (width 0.5) (layer F.Cu) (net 13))
 (segment (start 125.7 62) (end 129.5 62) (width 0.5) (layer F.Cu) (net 13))
 (via (at 125.7 62) (size 0.8) (drill 0.4) (layers F.Cu B.Cu) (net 13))
 (segment (start 132.55 66.5) (end 131.2 65.15) (width 0.5) (layer B.Cu) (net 13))
 (segment (start 133.4 66.5) (end 132.55 66.5) (width 0.5) (layer B.Cu) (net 13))
 (segment (start 129.5 63.45) (end 129.5 62) (width 0.5) (layer B.Cu) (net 13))
 (segment (start 131.2 65.15) (end 129.5 63.45) (width 0.5) (layer B.Cu) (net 13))
 (segment (start 119.300001 63.899999) (end 119.169999 63.899999) (width 0.5) (layer F.Cu) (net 13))
 (via (at 119.300001 63.899999) (size 0.8) (drill 0.4) (layers F.Cu B.Cu) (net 13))
 (segment (start 124.951459 63.899999) (end 119.300001 63.899999) (width 0.5) (layer F.Cu) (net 13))
 (segment (start 126.251458 62.6) (end 124.951459 63.899999) (width 0.5) (layer F.Cu) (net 13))
 (segment (start 127.9 62.6) (end 126.251458 62.6) (width 0.5) (layer F.Cu) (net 13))
 (segment (start 129.9 64.6) (end 127.9 62.6) (width 0.5) (layer F.Cu) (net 13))
 (segment (start 131.6 64.6) (end 129.9 64.6) (width 0.5) (layer F.Cu) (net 13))
 (segment (start 130.048 76.832) (end 128.72 78.16) (width 0.5) (layer F.Cu) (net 8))
 (segment (start 130.048 75.3488) (end 130.048 76.832) (width 0.5) (layer F.Cu) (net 8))
 (via (at 120.2 67.2) (size 0.8) (drill 0.4) (layers F.Cu B.Cu) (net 14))
 (segment (start 126.057603 73.993801) (end 122.393801 73.993801) (width 0.25) (layer F.Cu) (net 2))
 (segment (start 126.501801 74.437999) (end 126.057603 73.993801) (width 0.25) (layer F.Cu) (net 2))
 (segment (start 126.501801 76.298001) (end 126.501801 74.437999) (width 0.25) (layer F.Cu) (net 2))
 (segment (start 125.994999 78.690003) (end 125.994999 76.804803) (width 0.25) (layer F.Cu) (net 2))
 (segment (start 125.400001 79.285001) (end 125.994999 78.690003) (width 0.25) (layer F.Cu) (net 2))
 (segment (start 123.845001 79.285001) (end 125.400001 79.285001) (width 0.25) (layer F.Cu) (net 2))
 (segment (start 122.72 78.16) (end 123.845001 79.285001) (width 0.25) (layer F.Cu) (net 2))
 (segment (start 125.994999 76.804803) (end 126.501801 76.298001) (width 0.25) (layer F.Cu) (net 2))
 (segment (start 122.393801 73.993801) (end 122.2 73.8) (width 0.25) (layer F.Cu) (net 2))
 (segment (start 122.2 73.8) (end 122.2 70.3) (width 0.25) (layer F.Cu) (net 2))
 (segment (start 122.2 70.3) (end 122.2 70.3) (width 0.25) (layer F.Cu) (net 2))
 (via (at 122.2 70.3) (size 0.8) (drill 0.4) (layers F.Cu B.Cu) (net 2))
 (segment (start 122.2 68.15) (end 122.021 67.971) (width 0.25) (layer B.Cu) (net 2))
 (segment (start 122.2 70.3) (end 122.2 68.15) (width 0.25) (layer B.Cu) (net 2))
 (segment (start 122.021 67.971) (end 121.15 67.1) (width 0.25) (layer B.Cu) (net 2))
 (via (at 122.021 67.971) (size 0.5) (drill 0.3) (layers F.Cu B.Cu) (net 2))
 (segment (start 126.492 69.9268) (end 123.4 73.0188) (width 0.5) (layer F.Cu) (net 16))
 (segment (start 126.492 69.088) (end 126.492 69.9268) (width 0.5) (layer F.Cu) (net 16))
 (segment (start 123.4 75.48) (end 120.72 78.16) (width 0.5) (layer F.Cu) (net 5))
 (segment (start 123.4 75.4188) (end 123.4 75.48) (width 0.5) (layer F.Cu) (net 5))
 (via (at 117.8 62.5) (size 0.8) (drill 0.4) (layers F.Cu B.Cu) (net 17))
 (segment (start 121.15 63.45) (end 121.15 64.5) (width 0.5) (layer B.Cu) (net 12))
 (segment (start 120.3 62.6) (end 121.15 63.45) (width 0.5) (layer B.Cu) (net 12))
 (segment (start 121.15 64.5) (end 121.15 64.65) (width 0.5) (layer B.Cu) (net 12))
 (segment (start 121.825001 65.374999) (end 121.85 65.35) (width 0.5) (layer B.Cu) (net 12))
 (segment (start 121.85 65.35) (end 123 66.5) (width 0.5) (layer B.Cu) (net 12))
 (segment (start 121.15 64.65) (end 121.85 65.35) (width 0.5) (layer B.Cu) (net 12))
 (segment (start 123 66.5) (end 129.5 66.5) (width 0.5) (layer F.Cu) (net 12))
 (segment (start 120.5 72.6) (end 121.7 72.6) (width 0.5) (layer B.Cu) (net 12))
 (segment (start 123 71.3) (end 123 66.5) (width 0.5) (layer B.Cu) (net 12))
 (segment (start 121.7 72.6) (end 123 71.3) (width 0.5) (layer B.Cu) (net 12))
 (segment (start 120.550001 65.149999) (end 126.050001 65.149999) (width 0.5) (layer F.Cu) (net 15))
 (segment (start 120.3 65.4) (end 120.550001 65.149999) (width 0.5) (layer F.Cu) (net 15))
 (segment (start 126.050001 65.149999) (end 127.55 63.65) (width 0.5) (layer F.Cu) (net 15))
 (segment (start 127.55 63.65) (end 127.6 63.6) (width 0.5) (layer F.Cu) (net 15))
 (via (at 127.55 63.65) (size 0.8) (drill 0.4) (layers F.Cu B.Cu) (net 15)))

